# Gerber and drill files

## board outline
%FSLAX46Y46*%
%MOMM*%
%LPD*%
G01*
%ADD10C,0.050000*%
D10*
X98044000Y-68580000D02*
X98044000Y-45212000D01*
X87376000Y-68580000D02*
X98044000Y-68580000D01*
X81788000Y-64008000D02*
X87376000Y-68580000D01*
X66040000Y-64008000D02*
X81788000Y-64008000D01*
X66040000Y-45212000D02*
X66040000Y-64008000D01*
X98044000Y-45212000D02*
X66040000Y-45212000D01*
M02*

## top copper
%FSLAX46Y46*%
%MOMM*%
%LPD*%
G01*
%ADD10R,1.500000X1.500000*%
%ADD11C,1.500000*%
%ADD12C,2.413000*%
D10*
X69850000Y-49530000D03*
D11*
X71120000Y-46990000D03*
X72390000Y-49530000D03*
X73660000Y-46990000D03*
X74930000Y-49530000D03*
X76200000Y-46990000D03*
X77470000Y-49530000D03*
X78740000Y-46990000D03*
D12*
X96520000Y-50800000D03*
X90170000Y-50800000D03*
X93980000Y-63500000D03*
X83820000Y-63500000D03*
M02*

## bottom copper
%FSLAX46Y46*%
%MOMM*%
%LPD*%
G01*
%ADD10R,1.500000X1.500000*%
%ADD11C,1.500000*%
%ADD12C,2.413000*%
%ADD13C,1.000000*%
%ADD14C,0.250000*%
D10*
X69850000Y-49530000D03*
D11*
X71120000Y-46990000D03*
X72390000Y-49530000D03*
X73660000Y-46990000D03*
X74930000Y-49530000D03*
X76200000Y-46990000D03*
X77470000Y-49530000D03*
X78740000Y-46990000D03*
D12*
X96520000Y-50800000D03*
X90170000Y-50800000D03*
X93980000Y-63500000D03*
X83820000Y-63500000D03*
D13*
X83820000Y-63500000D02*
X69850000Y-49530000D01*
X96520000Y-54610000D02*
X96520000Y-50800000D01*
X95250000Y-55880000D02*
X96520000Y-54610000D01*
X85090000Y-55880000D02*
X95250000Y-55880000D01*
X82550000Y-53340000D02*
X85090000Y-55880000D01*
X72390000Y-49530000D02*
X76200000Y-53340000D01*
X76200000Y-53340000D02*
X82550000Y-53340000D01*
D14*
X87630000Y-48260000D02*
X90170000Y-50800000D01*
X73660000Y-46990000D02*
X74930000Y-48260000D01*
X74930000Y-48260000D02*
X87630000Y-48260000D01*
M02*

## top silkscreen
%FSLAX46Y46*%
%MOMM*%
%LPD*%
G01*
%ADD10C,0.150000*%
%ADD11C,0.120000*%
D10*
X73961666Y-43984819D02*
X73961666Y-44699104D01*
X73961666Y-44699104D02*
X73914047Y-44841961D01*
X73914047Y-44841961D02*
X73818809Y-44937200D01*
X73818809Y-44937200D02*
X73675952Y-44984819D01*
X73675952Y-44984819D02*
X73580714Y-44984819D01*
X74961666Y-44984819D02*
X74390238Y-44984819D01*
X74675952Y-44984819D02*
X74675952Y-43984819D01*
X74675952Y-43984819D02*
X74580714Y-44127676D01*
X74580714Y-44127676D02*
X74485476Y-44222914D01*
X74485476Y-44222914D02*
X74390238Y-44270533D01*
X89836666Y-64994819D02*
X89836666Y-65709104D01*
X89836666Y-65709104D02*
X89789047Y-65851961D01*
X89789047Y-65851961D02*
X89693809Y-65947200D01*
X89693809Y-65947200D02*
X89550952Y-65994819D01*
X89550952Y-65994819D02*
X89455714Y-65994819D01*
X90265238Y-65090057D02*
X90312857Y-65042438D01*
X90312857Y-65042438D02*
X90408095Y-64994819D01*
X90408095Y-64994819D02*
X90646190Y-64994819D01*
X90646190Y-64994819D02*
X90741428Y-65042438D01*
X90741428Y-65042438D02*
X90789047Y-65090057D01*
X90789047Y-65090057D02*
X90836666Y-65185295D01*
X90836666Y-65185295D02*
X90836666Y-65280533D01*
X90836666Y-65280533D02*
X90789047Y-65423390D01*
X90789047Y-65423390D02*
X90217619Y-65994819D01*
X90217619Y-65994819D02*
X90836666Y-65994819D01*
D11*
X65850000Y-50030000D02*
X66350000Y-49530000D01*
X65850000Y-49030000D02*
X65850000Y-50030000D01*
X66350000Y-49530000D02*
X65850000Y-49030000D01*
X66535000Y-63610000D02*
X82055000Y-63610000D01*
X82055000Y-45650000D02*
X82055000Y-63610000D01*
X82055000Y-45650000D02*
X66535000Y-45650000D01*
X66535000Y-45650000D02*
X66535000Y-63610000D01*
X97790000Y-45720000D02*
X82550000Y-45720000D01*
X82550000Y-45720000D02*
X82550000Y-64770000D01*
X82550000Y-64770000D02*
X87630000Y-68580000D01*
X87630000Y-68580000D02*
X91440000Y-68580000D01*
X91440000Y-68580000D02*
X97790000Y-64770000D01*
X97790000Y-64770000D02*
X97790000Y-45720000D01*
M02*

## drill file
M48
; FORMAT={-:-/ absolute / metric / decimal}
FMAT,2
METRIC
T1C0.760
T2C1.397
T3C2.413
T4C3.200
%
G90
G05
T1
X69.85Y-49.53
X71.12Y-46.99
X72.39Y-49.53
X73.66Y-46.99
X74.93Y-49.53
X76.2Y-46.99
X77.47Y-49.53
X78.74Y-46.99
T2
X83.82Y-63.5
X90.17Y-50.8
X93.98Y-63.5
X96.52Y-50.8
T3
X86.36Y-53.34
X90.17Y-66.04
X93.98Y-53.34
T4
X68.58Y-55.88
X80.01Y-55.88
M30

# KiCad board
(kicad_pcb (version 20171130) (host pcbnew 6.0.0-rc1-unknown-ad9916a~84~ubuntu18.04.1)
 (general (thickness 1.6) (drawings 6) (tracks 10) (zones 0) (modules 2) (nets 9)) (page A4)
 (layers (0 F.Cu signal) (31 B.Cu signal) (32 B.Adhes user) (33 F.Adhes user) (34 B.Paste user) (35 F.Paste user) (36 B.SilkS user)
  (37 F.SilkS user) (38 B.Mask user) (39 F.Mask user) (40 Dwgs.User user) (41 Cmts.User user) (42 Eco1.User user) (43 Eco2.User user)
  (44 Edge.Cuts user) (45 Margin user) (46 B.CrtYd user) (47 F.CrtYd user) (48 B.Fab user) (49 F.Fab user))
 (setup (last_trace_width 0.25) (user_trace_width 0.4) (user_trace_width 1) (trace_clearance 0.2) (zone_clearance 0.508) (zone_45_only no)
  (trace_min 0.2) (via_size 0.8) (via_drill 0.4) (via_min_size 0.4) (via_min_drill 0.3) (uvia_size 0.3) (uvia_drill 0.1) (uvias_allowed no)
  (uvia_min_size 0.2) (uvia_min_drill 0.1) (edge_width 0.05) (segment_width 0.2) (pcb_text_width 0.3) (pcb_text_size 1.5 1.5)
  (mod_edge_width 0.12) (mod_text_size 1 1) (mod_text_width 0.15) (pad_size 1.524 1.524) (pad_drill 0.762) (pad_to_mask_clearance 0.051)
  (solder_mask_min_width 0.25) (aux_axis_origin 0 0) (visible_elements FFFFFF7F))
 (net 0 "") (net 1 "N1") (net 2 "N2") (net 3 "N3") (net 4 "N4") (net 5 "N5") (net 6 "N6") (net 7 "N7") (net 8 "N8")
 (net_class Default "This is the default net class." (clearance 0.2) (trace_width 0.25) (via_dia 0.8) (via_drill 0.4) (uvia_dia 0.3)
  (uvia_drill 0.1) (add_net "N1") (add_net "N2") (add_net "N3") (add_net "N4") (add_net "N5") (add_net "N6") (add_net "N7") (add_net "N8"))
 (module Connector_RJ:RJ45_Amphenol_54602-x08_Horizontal (layer F.Cu) (at 69.85 49.53)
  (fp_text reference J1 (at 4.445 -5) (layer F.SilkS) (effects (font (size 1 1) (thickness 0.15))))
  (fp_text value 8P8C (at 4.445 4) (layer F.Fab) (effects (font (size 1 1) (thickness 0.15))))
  (fp_line (start -4 0.5) (end -3.5 0) (layer F.SilkS) (width 0.12))
  (fp_line (start -4 -0.5) (end -4 0.5) (layer F.SilkS) (width 0.12))
  (fp_line (start -3.5 0) (end -4 -0.5) (layer F.SilkS) (width 0.12))
  (fp_line (start -3.315 14.08) (end 12.205 14.08) (layer F.SilkS) (width 0.12))
  (fp_line (start 12.205 -3.88) (end 12.205 14.08) (layer F.SilkS) (width 0.12))
  (fp_line (start 12.205 -3.88) (end -3.315 -3.88) (layer F.SilkS) (width 0.12))
  (fp_line (start -3.315 -3.88) (end -3.315 14.08) (layer F.SilkS) (width 0.12))
  (pad "" np_thru_hole circle (at 10.16 6.35) (size 3.2 3.2) (drill 3.2) (layers *.Cu *.Mask))
  (pad "" np_thru_hole circle (at -1.27 6.35) (size 3.2 3.2) (drill 3.2) (layers *.Cu *.Mask))
  (pad 1 thru_hole rect (at 0 0) (size 1.5 1.5) (drill 0.76) (layers *.Cu *.Mask) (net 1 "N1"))
  (pad 2 thru_hole circle (at 1.27 -2.54) (size 1.5 1.5) (drill 0.76) (layers *.Cu *.Mask) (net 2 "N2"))
  (pad 3 thru_hole circle (at 2.54 0) (size 1.5 1.5) (drill 0.76) (layers *.Cu *.Mask) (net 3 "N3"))
  (pad 4 thru_hole circle (at 3.81 -2.54) (size 1.5 1.5) (drill 0.76) (layers *.Cu *.Mask) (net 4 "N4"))
  (pad 5 thru_hole circle (at 5.08 0) (size 1.5 1.5) (drill 0.76) (layers *.Cu *.Mask) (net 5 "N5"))
  (pad 6 thru_hole circle (at 6.35 -2.54) (size 1.5 1.5) (drill 0.76) (layers *.Cu *.Mask) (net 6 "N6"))
  (pad 7 thru_hole circle (at 7.62 0) (size 1.5 1.5) (drill 0.76) (layers *.Cu *.Mask) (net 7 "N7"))
  (pad 8 thru_hole circle (at 8.89 -2.54) (size 1.5 1.5) (drill 0.76) (layers *.Cu *.Mask) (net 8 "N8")))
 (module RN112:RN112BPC (layer F.Cu) (at 90.17 66.04 180)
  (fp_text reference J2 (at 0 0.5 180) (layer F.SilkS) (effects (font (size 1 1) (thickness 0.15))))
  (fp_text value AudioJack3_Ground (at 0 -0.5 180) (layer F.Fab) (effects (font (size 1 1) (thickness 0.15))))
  (fp_line (start -7.62 20.32) (end 7.62 20.32) (layer F.SilkS) (width 0.12))
  (fp_line (start 7.62 20.32) (end 7.62 1.27) (layer F.SilkS) (width 0.12))
  (fp_line (start 7.62 1.27) (end 2.54 -2.54) (layer F.SilkS) (width 0.12))
  (fp_line (start 2.54 -2.54) (end -1.27 -2.54) (layer F.SilkS) (width 0.12))
  (fp_line (start -1.27 -2.54) (end -7.62 1.27) (layer F.SilkS) (width 0.12))
  (fp_line (start -7.62 1.27) (end -7.62 20.32) (layer F.SilkS) (width 0.12))
  (pad "" np_thru_hole circle (at -3.81 12.7 180) (size 2.413 2.413) (drill 2.413) (layers *.Cu *.Mask))
  (pad "" np_thru_hole circle (at 3.81 12.7 180) (size 2.413 2.413) (drill 2.413) (layers *.Cu *.Mask))
  (pad "" np_thru_hole circle (at 0 0 180) (size 2.413 2.413) (drill 2.413) (layers *.Cu *.Mask))
  (pad R thru_hole circle (at -6.35 15.24 180) (size 2.413 2.413) (drill 1.397) (layers *.Cu *.Mask) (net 3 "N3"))
  (pad S thru_hole circle (at 0 15.24 180) (size 2.413 2.413) (drill 1.397) (layers *.Cu *.Mask) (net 4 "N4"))
  (pad G thru_hole circle (at -3.81 2.54 180) (size 2.413 2.413) (drill 1.397) (layers *.Cu *.Mask))
  (pad T thru_hole circle (at 6.35 2.54 180) (size 2.413 2.413) (drill 1.397) (layers *.Cu *.Mask) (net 1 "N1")))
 (gr_line (start 98.044 68.58) (end 98.044 45.212) (layer Edge.Cuts) (width 0.05))
 (gr_line (start 87.376 68.58) (end 98.044 68.58) (layer Edge.Cuts) (width 0.05))
 (gr_line (start 81.788 64.008) (end 87.376 68.58) (layer Edge.Cuts) (width 0.05))
 (gr_line (start 66.04 64.008) (end 81.788 64.008) (layer Edge.Cuts) (width 0.05))
 (gr_line (start 66.04 45.212) (end 66.04 64.008) (layer Edge.Cuts) (width 0.05))
 (gr_line (start 98.044 45.212) (end 66.04 45.212) (layer Edge.Cuts) (width 0.05))
 (segment (start 83.82 63.5) (end 69.85 49.53) (width 1) (layer B.Cu) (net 1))
 (segment (start 96.52 54.61) (end 96.52 50.8) (width 1) (layer B.Cu) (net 3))
 (segment (start 95.25 55.88) (end 96.52 54.61) (width 1) (layer B.Cu) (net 3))
 (segment (start 85.09 55.88) (end 95.25 55.88) (width 1) (layer B.Cu) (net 3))
 (segment (start 82.55 53.34) (end 85.09 55.88) (width 1) (layer B.Cu) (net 3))
 (segment (start 72.39 49.53) (end 76.2 53.34) (width 1) (layer B.Cu) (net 3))
 (segment (start 76.2 53.34) (end 82.55 53.34) (width 1) (layer B.Cu) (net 3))
 (segment (start 87.63 48.26) (end 90.17 50.8) (width 0.25) (layer B.Cu) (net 4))
 (segment (start 73.66 46.99) (end 74.93 48.26) (width 0.25) (layer B.Cu) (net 4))
 (segment (start 74.93 48.26) (end 87.63 48.26) (width 0.25) (layer B.Cu) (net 4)))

